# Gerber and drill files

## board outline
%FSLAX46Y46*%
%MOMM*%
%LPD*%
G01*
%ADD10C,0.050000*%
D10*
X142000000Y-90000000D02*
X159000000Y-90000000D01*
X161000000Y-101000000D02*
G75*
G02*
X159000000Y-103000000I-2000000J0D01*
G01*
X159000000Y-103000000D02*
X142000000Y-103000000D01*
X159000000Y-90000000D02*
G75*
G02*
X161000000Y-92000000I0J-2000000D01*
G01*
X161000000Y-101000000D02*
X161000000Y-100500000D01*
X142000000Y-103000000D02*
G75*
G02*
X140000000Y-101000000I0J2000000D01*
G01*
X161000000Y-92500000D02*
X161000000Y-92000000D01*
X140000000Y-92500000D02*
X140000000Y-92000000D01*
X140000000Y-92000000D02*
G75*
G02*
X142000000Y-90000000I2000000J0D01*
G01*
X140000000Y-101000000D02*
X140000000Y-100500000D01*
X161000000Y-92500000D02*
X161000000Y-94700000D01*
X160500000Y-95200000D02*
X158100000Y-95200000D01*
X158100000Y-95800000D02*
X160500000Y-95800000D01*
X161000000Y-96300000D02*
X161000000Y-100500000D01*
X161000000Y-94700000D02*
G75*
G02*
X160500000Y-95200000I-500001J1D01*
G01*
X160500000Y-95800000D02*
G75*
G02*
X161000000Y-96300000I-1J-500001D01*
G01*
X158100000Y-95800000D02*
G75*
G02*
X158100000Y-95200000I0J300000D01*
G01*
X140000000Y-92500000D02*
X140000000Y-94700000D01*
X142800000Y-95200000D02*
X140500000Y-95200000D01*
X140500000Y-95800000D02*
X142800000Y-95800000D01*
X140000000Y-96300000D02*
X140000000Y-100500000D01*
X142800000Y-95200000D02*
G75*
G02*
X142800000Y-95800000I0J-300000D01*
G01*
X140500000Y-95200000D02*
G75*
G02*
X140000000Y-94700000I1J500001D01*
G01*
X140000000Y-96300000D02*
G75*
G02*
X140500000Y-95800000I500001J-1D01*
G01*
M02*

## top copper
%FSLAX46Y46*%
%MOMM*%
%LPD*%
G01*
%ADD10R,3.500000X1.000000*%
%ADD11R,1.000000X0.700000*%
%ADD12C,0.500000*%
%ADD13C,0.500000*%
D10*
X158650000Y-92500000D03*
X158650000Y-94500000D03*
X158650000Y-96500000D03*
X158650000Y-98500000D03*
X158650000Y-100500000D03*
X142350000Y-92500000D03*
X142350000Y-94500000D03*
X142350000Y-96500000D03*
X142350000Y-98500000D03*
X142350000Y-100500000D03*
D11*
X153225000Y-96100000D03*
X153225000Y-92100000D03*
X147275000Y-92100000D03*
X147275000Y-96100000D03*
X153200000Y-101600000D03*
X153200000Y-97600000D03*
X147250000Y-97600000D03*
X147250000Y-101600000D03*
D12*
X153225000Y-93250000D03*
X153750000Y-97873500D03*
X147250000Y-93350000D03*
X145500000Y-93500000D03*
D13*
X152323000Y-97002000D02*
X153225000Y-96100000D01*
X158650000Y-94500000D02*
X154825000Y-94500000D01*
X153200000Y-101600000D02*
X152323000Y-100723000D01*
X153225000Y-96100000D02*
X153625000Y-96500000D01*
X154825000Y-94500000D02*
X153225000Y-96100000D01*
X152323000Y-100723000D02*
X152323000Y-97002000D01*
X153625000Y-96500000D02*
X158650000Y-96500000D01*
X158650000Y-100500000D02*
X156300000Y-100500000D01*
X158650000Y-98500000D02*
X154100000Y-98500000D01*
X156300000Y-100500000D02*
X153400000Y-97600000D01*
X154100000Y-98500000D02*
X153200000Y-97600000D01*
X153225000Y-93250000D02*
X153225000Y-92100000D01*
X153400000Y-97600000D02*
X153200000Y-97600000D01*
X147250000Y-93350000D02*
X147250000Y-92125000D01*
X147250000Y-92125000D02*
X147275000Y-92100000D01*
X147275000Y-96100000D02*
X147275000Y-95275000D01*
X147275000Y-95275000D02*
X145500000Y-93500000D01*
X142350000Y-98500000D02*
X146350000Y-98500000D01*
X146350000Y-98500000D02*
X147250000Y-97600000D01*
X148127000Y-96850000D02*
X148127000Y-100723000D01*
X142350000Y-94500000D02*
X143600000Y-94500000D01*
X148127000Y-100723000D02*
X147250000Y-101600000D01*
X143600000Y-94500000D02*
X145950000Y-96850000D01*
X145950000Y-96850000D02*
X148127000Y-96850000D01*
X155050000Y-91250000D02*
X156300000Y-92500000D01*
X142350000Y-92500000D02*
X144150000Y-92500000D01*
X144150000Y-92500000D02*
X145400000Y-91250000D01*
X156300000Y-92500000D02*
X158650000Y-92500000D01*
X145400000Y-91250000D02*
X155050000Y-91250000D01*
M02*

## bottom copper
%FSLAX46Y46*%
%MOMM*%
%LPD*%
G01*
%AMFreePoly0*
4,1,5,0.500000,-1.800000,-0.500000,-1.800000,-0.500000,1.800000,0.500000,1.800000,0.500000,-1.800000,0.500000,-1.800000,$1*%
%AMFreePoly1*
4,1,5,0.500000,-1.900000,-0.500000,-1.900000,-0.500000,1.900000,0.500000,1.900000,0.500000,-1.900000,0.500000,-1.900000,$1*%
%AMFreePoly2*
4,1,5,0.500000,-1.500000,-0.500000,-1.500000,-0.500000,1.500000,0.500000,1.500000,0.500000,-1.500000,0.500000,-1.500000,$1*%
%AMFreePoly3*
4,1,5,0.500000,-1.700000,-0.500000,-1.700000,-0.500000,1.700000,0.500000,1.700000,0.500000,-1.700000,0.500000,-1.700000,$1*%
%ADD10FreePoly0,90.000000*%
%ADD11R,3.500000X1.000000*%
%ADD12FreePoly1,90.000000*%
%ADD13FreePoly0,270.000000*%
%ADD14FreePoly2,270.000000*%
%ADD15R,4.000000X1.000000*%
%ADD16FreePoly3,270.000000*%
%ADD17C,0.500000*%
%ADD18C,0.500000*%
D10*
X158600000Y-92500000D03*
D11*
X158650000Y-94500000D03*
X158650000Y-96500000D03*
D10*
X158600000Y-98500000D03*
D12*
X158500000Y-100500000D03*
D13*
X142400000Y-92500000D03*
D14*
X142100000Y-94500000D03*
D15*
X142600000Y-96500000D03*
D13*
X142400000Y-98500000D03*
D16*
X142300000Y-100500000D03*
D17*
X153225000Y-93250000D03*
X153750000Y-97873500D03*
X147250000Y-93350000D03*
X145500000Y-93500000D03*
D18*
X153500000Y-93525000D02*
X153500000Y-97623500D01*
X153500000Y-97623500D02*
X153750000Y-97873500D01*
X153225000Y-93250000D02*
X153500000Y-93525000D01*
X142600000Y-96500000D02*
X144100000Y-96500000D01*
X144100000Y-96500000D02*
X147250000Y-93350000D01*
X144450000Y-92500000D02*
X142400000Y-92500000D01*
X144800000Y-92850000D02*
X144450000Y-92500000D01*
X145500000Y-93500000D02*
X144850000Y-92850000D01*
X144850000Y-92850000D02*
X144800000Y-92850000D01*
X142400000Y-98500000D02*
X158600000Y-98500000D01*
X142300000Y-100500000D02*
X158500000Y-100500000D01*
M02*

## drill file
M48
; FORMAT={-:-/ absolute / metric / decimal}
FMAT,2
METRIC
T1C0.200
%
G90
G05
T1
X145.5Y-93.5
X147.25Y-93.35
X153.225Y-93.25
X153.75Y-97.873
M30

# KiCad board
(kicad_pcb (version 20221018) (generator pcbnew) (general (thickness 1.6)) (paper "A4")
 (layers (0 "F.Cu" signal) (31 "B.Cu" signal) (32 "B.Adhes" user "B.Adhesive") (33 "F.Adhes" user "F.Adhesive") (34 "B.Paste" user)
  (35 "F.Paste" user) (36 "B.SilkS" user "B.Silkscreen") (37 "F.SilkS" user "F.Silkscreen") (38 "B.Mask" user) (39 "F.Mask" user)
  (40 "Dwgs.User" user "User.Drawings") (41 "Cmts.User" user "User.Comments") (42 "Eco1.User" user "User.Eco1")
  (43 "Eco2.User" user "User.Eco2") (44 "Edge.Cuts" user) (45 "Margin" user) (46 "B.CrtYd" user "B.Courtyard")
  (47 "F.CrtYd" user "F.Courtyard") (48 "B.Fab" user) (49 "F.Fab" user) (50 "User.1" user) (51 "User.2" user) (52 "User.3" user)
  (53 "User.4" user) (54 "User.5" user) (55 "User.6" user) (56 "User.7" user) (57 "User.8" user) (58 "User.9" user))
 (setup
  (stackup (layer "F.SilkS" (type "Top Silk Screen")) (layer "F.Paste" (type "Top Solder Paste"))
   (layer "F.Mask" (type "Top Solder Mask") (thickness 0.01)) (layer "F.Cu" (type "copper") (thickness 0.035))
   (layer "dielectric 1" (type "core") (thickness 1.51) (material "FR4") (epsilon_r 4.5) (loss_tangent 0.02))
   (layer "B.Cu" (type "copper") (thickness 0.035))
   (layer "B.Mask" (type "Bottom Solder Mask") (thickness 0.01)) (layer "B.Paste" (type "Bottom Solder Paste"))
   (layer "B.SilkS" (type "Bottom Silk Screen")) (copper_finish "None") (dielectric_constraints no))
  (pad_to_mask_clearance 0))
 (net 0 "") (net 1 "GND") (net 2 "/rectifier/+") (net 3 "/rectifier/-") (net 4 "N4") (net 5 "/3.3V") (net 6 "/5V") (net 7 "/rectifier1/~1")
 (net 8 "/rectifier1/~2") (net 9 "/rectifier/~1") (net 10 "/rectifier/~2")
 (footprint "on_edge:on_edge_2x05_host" (layer "F.Cu") (at 161 96.5 -90)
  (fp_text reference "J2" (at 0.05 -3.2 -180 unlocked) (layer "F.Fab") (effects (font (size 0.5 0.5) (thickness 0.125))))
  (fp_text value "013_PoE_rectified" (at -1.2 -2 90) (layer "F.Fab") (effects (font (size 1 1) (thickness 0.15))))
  (fp_line (start -4 0) (end -1.8 0) (stroke (width 0.05) (type solid)) (layer "Edge.Cuts"))
  (fp_line (start -1.3 0.5) (end -1.3 2.9) (stroke (width 0.05) (type solid)) (layer "Edge.Cuts"))
  (fp_line (start -0.7 2.9) (end -0.7 0.5) (stroke (width 0.05) (type solid)) (layer "Edge.Cuts"))
  (fp_line (start -0.2 0) (end 4 0) (stroke (width 0.05) (type solid)) (layer "Edge.Cuts"))
  (fp_arc (start -1.8 0) (mid -1.446447 0.146447) (end -1.3 0.5) (stroke (width 0.05) (type solid)) (layer "Edge.Cuts"))
  (fp_arc (start -0.7 0.5) (mid -0.553553 0.146447) (end -0.2 0) (stroke (width 0.05) (type solid)) (layer "Edge.Cuts"))
  (fp_arc (start -0.7 2.9) (mid -1 3.2) (end -1.3 2.9) (stroke (width 0.05) (type solid)) (layer "Edge.Cuts"))
  (pad "1" smd rect (at -4 2.35 270) (size 1 3.5) (layers "F.Cu" "F.Mask") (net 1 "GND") (zone_connect 0))
  (pad "2" smd rect (at -2 2.35 270) (size 1 3.5) (layers "F.Cu" "F.Mask") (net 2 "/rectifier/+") (zone_connect 0))
  (pad "3" smd rect (at 0 2.35 270) (size 1 3.5) (layers "F.Cu" "F.Mask") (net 2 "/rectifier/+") (zone_connect 0))
  (pad "4" smd rect (at 2 2.35 270) (size 1 3.5) (layers "F.Cu" "F.Mask") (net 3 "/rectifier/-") (zone_connect 0))
  (pad "5" smd rect (at 4 2.35 270) (size 1 3.5) (layers "F.Cu" "F.Mask") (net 3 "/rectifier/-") (zone_connect 0))
  (pad "6" smd custom (at -4 2.4 90) (size 1 3.6) (layers "B.Cu" "B.Mask") (zone_connect 0) (options (clearance outline) (anchor rect))
   (primitives))
  (pad "7" smd rect (at -2 2.35 90) (size 1 3.5) (layers "B.Cu" "B.Mask") (zone_connect 0))
  (pad "8" smd rect (at 0 2.35 90) (size 1 3.5) (layers "B.Cu" "B.Mask") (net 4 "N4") (zone_connect 0))
  (pad "9" smd custom (at 2 2.4 90) (size 1 3.6) (layers "B.Cu" "B.Mask") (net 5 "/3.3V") (zone_connect 0)
   (options (clearance outline) (anchor rect)) (primitives))
  (pad "10" smd custom (at 4 2.5 90) (size 1 3.8) (layers "B.Cu" "B.Mask") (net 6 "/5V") (zone_connect 0)
   (options (clearance outline) (anchor rect)) (primitives))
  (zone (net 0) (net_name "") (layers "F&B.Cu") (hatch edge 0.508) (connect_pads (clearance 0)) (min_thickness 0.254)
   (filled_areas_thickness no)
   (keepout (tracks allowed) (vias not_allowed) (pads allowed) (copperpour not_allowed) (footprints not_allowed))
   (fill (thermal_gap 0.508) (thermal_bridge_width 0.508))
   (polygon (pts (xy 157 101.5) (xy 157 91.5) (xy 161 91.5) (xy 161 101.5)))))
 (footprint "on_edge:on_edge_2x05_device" (layer "F.Cu") (at 140 96.5 -90)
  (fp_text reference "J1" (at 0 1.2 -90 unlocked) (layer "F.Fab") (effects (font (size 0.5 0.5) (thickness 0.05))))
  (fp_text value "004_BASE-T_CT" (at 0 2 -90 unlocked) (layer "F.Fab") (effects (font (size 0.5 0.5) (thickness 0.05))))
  (fp_line (start -4 0) (end -1.8 0) (stroke (width 0.05) (type solid)) (layer "Edge.Cuts"))
  (fp_line (start -1.3 -2.8) (end -1.3 -0.5) (stroke (width 0.05) (type solid)) (layer "Edge.Cuts"))
  (fp_line (start -0.7 -0.5) (end -0.7 -2.8) (stroke (width 0.05) (type solid)) (layer "Edge.Cuts"))
  (fp_line (start -0.2 0) (end 4 0) (stroke (width 0.05) (type solid)) (layer "Edge.Cuts"))
  (fp_arc (start -1.3 -2.8) (mid -1 -3.1) (end -0.7 -2.8) (stroke (width 0.05) (type solid)) (layer "Edge.Cuts"))
  (fp_arc (start -1.3 -0.5) (mid -1.446447 -0.146447) (end -1.8 0) (stroke (width 0.05) (type solid)) (layer "Edge.Cuts"))
  (fp_arc (start -0.2 0) (mid -0.553553 -0.146447) (end -0.7 -0.5) (stroke (width 0.05) (type solid)) (layer "Edge.Cuts"))
  (pad "1" smd rect (at -4 -2.35 90) (size 1 3.5) (layers "F.Cu" "F.Mask") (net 1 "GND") (zone_connect 0))
  (pad "2" smd rect (at -2 -2.35 270) (size 1 3.5) (layers "F.Cu" "F.Mask") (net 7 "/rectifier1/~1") (zone_connect 0))
  (pad "3" smd rect (at 0 -2.35 270) (size 1 3.5) (layers "F.Cu" "F.Mask") (zone_connect 0))
  (pad "4" smd rect (at 2 -2.35 90) (size 1 3.5) (layers "F.Cu" "F.Mask") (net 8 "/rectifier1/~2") (zone_connect 0))
  (pad "5" smd rect (at 4 -2.35 90) (size 1 3.5) (layers "F.Cu" "F.Mask") (zone_connect 0))
  (pad "6" smd custom (at -4 -2.4 270) (size 1 3.6) (layers "B.Cu" "B.Mask") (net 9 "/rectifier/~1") (zone_connect 0)
   (options (clearance outline) (anchor rect)) (primitives))
  (pad "7" smd custom (at -2 -2.1 270) (size 1 3) (layers "B.Cu" "B.Mask") (zone_connect 0) (options (clearance outline) (anchor rect))
   (primitives))
  (pad "8" smd rect (at 0 -2.6 270) (size 1 4) (layers "B.Cu" "B.Mask") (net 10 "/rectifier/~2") (zone_connect 0))
  (pad "9" smd custom (at 2 -2.4 270) (size 1 3.6) (layers "B.Cu" "B.Mask") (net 5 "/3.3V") (zone_connect 0)
   (options (clearance outline) (anchor rect)) (primitives))
  (pad "10" smd custom (at 4 -2.3 270) (size 1 3.4) (layers "B.Cu" "B.Mask") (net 6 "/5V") (zone_connect 0)
   (options (clearance outline) (anchor rect)) (primitives))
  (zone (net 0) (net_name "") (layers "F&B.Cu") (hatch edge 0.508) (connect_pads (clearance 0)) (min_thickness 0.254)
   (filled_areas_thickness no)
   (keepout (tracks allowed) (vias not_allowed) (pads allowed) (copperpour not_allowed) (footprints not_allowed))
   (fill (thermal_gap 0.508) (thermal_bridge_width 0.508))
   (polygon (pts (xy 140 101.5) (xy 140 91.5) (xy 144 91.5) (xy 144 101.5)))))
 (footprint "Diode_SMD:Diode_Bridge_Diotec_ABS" (layer "F.Cu") (at 150.25 94.1 180)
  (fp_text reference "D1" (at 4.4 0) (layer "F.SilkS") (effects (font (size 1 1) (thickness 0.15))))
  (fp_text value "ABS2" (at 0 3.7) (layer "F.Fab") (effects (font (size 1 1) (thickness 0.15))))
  (pad "1" smd rect (at -2.975 -2 180) (size 1 0.7) (layers "F.Cu" "F.Paste" "F.Mask") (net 2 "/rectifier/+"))
  (pad "2" smd rect (at -2.975 2 180) (size 1 0.7) (layers "F.Cu" "F.Paste" "F.Mask") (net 3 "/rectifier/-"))
  (pad "3" smd rect (at 2.975 2 180) (size 1 0.7) (layers "F.Cu" "F.Paste" "F.Mask") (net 10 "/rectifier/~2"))
  (pad "4" smd rect (at 2.975 -2 180) (size 1 0.7) (layers "F.Cu" "F.Paste" "F.Mask") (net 9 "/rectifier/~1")))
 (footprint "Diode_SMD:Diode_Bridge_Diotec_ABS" (layer "F.Cu") (at 150.225 99.6 180)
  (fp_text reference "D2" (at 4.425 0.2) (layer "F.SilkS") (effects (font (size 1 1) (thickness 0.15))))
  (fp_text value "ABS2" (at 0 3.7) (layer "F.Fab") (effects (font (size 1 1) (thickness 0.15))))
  (pad "1" smd rect (at -2.975 -2 180) (size 1 0.7) (layers "F.Cu" "F.Paste" "F.Mask") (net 2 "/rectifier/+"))
  (pad "2" smd rect (at -2.975 2 180) (size 1 0.7) (layers "F.Cu" "F.Paste" "F.Mask") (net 3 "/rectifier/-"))
  (pad "3" smd rect (at 2.975 2 180) (size 1 0.7) (layers "F.Cu" "F.Paste" "F.Mask") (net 8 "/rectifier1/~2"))
  (pad "4" smd rect (at 2.975 -2 180) (size 1 0.7) (layers "F.Cu" "F.Paste" "F.Mask") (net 7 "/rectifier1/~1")))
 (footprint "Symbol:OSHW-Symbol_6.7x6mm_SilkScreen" (layer "B.Cu") (at 150 99 180)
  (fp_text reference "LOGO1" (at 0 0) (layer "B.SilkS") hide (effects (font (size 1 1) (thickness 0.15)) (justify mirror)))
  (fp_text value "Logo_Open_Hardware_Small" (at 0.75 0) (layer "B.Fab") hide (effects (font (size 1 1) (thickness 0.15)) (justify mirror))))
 (gr_line (start 142 90) (end 159 90) (stroke (width 0.05) (type solid)) (layer "Edge.Cuts"))
 (gr_arc (start 161 101) (mid 160.414214 102.414214) (end 159 103) (stroke (width 0.05) (type solid)) (layer "Edge.Cuts"))
 (gr_line (start 159 103) (end 142 103) (stroke (width 0.05) (type solid)) (layer "Edge.Cuts"))
 (gr_arc (start 159 90) (mid 160.414214 90.585786) (end 161 92) (stroke (width 0.05) (type solid)) (layer "Edge.Cuts"))
 (gr_line (start 161 101) (end 161 100.5) (stroke (width 0.05) (type default)) (layer "Edge.Cuts"))
 (gr_arc (start 142 103) (mid 140.585786 102.414214) (end 140 101) (stroke (width 0.05) (type solid)) (layer "Edge.Cuts"))
 (gr_line (start 161 92.5) (end 161 92) (stroke (width 0.05) (type solid)) (layer "Edge.Cuts"))
 (gr_line (start 140 92.5) (end 140 92) (stroke (width 0.05) (type solid)) (layer "Edge.Cuts"))
 (gr_arc (start 140 92) (mid 140.585786 90.585786) (end 142 90) (stroke (width 0.05) (type solid)) (layer "Edge.Cuts"))
 (gr_line (start 140 101) (end 140 100.5) (stroke (width 0.05) (type default)) (layer "Edge.Cuts"))
 (segment (start 152.323 97.002) (end 153.225 96.1) (width 0.5) (layer "F.Cu") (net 2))
 (segment (start 158.65 94.5) (end 154.825 94.5) (width 0.5) (layer "F.Cu") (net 2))
 (segment (start 153.2 101.6) (end 152.323 100.723) (width 0.5) (layer "F.Cu") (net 2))
 (segment (start 153.225 96.1) (end 153.625 96.5) (width 0.5) (layer "F.Cu") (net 2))
 (segment (start 154.825 94.5) (end 153.225 96.1) (width 0.5) (layer "F.Cu") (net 2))
 (segment (start 152.323 100.723) (end 152.323 97.002) (width 0.5) (layer "F.Cu") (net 2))
 (segment (start 153.625 96.5) (end 158.65 96.5) (width 0.5) (layer "F.Cu") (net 2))
 (segment (start 158.65 100.5) (end 156.3 100.5) (width 0.5) (layer "F.Cu") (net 3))
 (segment (start 158.65 98.5) (end 154.1 98.5) (width 0.5) (layer "F.Cu") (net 3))
 (segment (start 156.3 100.5) (end 153.4 97.6) (width 0.5) (layer "F.Cu") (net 3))
 (segment (start 154.1 98.5) (end 153.2 97.6) (width 0.5) (layer "F.Cu") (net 3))
 (segment (start 153.225 93.25) (end 153.225 92.1) (width 0.5) (layer "F.Cu") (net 3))
 (segment (start 153.4 97.6) (end 153.2 97.6) (width 0.5) (layer "F.Cu") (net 3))
 (via (at 153.225 93.25) (size 0.5) (drill 0.2) (layers "F.Cu" "B.Cu") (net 3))
 (via (at 153.75 97.8735) (size 0.5) (drill 0.2) (layers "F.Cu" "B.Cu") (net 3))
 (segment (start 153.5 93.525) (end 153.5 97.6235) (width 0.5) (layer "B.Cu") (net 3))
 (segment (start 153.5 97.6235) (end 153.75 97.8735) (width 0.5) (layer "B.Cu") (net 3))
 (segment (start 153.225 93.25) (end 153.5 93.525) (width 0.5) (layer "B.Cu") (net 3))
 (segment (start 147.25 93.35) (end 147.25 92.125) (width 0.5) (layer "F.Cu") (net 10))
 (segment (start 147.25 92.125) (end 147.275 92.1) (width 0.5) (layer "F.Cu") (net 10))
 (via (at 147.25 93.35) (size 0.5) (drill 0.2) (layers "F.Cu" "B.Cu") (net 10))
 (segment (start 142.6 96.5) (end 144.1 96.5) (width 0.5) (layer "B.Cu") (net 10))
 (segment (start 144.1 96.5) (end 147.25 93.35) (width 0.5) (layer "B.Cu") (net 10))
 (segment (start 147.275 96.1) (end 147.275 95.275) (width 0.5) (layer "F.Cu") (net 9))
 (segment (start 147.275 95.275) (end 145.5 93.5) (width 0.5) (layer "F.Cu") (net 9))
 (via (at 145.5 93.5) (size 0.5) (drill 0.2) (layers "F.Cu" "B.Cu") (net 9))
 (segment (start 144.45 92.5) (end 142.4 92.5) (width 0.5) (layer "B.Cu") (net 9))
 (segment (start 144.8 92.85) (end 144.45 92.5) (width 0.5) (layer "B.Cu") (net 9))
 (segment (start 145.5 93.5) (end 144.85 92.85) (width 0.5) (layer "B.Cu") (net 9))
 (segment (start 144.85 92.85) (end 144.8 92.85) (width 0.5) (layer "B.Cu") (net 9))
 (segment (start 142.35 98.5) (end 146.35 98.5) (width 0.5) (layer "F.Cu") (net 8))
 (segment (start 146.35 98.5) (end 147.25 97.6) (width 0.5) (layer "F.Cu") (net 8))
 (segment (start 148.127 96.85) (end 148.127 100.723) (width 0.5) (layer "F.Cu") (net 7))
 (segment (start 142.35 94.5) (end 143.6 94.5) (width 0.5) (layer "F.Cu") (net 7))
 (segment (start 148.127 100.723) (end 147.25 101.6) (width 0.5) (layer "F.Cu") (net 7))
 (segment (start 143.6 94.5) (end 145.95 96.85) (width 0.5) (layer "F.Cu") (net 7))
 (segment (start 145.95 96.85) (end 148.127 96.85) (width 0.5) (layer "F.Cu") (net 7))
 (segment (start 155.05 91.25) (end 156.3 92.5) (width 0.5) (layer "F.Cu") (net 1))
 (segment (start 142.35 92.5) (end 144.15 92.5) (width 0.5) (layer "F.Cu") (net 1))
 (segment (start 144.15 92.5) (end 145.4 91.25) (width 0.5) (layer "F.Cu") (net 1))
 (segment (start 156.3 92.5) (end 158.65 92.5) (width 0.5) (layer "F.Cu") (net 1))
 (segment (start 145.4 91.25) (end 155.05 91.25) (width 0.5) (layer "F.Cu") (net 1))
 (segment (start 142.4 98.5) (end 158.6 98.5) (width 0.5) (layer "B.Cu") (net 5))
 (segment (start 142.3 100.5) (end 158.5 100.5) (width 0.5) (layer "B.Cu") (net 6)))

